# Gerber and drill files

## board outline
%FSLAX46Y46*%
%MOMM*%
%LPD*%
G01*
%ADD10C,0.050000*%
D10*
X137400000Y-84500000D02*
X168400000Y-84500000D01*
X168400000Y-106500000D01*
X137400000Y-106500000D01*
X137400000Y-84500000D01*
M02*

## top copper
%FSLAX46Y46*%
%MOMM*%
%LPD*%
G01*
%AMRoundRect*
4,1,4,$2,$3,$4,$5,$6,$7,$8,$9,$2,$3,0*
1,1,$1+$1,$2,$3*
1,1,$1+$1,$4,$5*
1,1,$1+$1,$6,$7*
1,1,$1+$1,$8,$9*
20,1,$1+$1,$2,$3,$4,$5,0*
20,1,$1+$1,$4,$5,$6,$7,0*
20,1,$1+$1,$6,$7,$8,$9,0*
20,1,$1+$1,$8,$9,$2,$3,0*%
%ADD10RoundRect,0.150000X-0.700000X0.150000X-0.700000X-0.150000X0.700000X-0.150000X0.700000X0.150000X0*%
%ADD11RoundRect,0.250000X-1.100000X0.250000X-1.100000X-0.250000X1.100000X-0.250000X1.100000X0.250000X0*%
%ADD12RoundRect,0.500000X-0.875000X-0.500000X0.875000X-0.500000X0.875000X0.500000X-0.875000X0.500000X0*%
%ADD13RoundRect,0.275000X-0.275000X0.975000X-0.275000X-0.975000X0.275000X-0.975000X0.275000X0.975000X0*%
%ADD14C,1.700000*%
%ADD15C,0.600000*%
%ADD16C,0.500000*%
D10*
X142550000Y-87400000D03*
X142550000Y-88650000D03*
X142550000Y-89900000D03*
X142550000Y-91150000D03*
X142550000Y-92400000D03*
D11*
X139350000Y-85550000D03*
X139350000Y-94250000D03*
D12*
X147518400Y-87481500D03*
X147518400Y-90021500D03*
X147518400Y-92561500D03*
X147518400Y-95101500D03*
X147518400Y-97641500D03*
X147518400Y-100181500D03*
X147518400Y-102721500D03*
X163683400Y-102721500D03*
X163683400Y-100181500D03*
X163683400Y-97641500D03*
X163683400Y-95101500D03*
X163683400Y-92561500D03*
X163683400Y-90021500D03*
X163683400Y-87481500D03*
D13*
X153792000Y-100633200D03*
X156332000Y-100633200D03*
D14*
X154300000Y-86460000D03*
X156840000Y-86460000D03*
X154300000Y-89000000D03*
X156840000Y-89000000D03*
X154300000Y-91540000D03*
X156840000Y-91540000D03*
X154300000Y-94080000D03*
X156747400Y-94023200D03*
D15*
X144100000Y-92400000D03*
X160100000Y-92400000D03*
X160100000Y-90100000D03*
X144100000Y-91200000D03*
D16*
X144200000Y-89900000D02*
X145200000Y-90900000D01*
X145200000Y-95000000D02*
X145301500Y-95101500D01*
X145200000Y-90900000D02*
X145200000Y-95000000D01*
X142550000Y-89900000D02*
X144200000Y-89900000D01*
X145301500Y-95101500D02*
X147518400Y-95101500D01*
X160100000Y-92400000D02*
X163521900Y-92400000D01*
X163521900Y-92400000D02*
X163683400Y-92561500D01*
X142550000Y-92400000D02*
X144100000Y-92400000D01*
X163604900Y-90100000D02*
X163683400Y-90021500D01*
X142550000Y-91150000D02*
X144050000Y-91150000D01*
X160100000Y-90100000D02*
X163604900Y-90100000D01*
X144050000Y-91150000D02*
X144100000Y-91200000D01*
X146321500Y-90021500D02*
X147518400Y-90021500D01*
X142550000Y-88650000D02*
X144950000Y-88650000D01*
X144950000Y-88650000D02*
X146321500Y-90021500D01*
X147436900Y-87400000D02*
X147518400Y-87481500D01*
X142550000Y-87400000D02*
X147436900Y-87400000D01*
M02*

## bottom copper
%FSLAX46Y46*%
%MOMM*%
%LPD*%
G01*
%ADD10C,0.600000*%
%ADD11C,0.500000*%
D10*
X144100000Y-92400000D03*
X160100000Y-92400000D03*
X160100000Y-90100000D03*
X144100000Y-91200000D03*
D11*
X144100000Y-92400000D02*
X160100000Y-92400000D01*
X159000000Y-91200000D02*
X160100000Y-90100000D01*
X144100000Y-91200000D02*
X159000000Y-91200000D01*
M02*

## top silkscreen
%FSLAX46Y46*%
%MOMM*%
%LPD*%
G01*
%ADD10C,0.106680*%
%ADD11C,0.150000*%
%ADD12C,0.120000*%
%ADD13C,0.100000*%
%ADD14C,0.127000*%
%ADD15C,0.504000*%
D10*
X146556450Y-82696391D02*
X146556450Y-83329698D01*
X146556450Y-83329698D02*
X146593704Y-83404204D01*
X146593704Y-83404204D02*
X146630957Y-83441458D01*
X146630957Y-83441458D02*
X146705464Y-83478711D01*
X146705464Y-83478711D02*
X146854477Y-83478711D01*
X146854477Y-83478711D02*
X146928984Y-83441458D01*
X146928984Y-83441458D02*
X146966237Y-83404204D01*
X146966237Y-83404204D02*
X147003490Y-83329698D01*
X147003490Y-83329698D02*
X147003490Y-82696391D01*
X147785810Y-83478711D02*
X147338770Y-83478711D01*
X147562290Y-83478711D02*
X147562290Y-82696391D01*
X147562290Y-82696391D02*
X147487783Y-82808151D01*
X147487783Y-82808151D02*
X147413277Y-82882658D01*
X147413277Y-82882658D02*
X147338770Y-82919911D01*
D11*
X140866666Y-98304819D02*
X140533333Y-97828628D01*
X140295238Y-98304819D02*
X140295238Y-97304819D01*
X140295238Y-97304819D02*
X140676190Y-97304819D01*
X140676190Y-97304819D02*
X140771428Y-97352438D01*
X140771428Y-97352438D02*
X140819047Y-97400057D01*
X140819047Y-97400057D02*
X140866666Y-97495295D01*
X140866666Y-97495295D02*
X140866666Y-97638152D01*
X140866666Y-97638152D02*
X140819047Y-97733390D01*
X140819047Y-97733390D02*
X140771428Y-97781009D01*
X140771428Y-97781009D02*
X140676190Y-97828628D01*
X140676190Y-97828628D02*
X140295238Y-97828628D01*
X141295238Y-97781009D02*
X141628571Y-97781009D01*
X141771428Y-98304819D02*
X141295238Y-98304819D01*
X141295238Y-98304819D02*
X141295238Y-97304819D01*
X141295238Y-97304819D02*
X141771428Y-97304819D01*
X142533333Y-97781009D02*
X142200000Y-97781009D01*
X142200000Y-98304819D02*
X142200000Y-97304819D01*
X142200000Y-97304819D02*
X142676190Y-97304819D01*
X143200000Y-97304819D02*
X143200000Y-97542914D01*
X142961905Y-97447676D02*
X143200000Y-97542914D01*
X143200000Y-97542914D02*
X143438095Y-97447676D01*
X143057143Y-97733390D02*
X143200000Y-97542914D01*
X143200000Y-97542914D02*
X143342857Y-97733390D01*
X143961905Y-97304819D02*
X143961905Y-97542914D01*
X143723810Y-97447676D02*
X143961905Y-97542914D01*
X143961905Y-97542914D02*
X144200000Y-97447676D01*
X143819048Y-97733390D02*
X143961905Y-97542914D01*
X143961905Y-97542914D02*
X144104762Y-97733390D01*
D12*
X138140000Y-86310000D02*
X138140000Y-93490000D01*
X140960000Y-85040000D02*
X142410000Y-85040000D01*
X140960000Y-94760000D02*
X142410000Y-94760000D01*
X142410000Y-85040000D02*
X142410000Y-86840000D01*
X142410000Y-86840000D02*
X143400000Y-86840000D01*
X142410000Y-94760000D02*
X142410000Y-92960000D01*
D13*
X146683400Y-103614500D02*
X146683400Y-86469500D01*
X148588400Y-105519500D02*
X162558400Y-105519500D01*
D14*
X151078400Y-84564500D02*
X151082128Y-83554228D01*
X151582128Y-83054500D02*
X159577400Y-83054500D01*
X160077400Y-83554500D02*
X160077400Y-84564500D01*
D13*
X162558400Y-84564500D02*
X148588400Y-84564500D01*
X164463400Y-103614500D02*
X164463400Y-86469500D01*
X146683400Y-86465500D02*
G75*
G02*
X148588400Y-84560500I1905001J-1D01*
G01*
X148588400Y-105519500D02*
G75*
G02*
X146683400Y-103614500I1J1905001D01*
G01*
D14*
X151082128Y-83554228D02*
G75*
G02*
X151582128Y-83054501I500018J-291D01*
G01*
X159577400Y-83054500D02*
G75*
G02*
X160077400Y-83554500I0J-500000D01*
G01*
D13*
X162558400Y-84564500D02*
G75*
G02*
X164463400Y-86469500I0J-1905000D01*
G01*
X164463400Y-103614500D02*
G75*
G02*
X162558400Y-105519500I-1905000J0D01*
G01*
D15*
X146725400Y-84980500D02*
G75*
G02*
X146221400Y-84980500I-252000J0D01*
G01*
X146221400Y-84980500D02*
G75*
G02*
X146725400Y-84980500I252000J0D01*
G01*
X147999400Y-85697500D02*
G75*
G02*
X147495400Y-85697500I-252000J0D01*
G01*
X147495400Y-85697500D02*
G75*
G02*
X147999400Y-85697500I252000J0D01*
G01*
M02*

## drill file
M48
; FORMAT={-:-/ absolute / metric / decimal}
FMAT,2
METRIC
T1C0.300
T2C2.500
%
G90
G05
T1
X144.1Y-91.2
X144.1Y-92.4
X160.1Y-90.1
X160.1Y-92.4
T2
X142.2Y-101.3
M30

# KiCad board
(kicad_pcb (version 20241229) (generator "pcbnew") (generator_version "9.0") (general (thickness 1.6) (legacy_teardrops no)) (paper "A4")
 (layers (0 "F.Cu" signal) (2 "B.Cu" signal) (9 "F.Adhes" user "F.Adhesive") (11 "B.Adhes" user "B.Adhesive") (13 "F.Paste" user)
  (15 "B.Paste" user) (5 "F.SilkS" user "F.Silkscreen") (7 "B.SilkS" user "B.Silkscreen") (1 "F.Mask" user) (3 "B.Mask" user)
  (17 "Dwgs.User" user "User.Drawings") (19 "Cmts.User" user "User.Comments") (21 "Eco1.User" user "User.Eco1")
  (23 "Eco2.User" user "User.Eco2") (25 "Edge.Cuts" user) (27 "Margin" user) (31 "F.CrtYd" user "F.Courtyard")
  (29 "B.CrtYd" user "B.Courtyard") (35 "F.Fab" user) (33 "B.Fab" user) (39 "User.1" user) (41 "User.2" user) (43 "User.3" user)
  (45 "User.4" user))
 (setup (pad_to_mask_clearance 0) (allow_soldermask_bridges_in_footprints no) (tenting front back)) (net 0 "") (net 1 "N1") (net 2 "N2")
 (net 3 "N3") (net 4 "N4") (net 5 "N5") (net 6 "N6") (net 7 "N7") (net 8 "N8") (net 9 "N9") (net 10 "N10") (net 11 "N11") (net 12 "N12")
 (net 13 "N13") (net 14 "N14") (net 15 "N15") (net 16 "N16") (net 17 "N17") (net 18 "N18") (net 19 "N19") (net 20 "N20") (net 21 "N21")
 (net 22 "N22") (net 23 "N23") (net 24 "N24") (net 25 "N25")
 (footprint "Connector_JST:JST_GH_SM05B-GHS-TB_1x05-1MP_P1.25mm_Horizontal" (layer "F.Cu") (at 140.7 89.9 -90)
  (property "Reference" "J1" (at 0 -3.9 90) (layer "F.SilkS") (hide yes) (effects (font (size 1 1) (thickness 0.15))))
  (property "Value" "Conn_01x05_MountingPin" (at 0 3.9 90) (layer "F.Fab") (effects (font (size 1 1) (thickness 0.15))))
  (fp_line (start -3.59 2.56) (end 3.59 2.56) (stroke (width 0.12) (type solid)) (layer "F.SilkS"))
  (fp_line (start -4.86 -0.26) (end -4.86 -1.71) (stroke (width 0.12) (type solid)) (layer "F.SilkS"))
  (fp_line (start 4.86 -0.26) (end 4.86 -1.71) (stroke (width 0.12) (type solid)) (layer "F.SilkS"))
  (fp_line (start -4.86 -1.71) (end -3.06 -1.71) (stroke (width 0.12) (type solid)) (layer "F.SilkS"))
  (fp_line (start -3.06 -1.71) (end -3.06 -2.7) (stroke (width 0.12) (type solid)) (layer "F.SilkS"))
  (fp_line (start 4.86 -1.71) (end 3.06 -1.71) (stroke (width 0.12) (type solid)) (layer "F.SilkS"))
  (pad "1" smd roundrect (at -2.5 -1.85 270) (size 0.6 1.7) (layers "F.Cu" "F.Mask" "F.Paste") (roundrect_rratio 0.25) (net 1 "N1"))
  (pad "2" smd roundrect (at -1.25 -1.85 270) (size 0.6 1.7) (layers "F.Cu" "F.Mask" "F.Paste") (roundrect_rratio 0.25) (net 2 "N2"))
  (pad "3" smd roundrect (at 0 -1.85 270) (size 0.6 1.7) (layers "F.Cu" "F.Mask" "F.Paste") (roundrect_rratio 0.25) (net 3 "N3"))
  (pad "4" smd roundrect (at 1.25 -1.85 270) (size 0.6 1.7) (layers "F.Cu" "F.Mask" "F.Paste") (roundrect_rratio 0.25) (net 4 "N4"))
  (pad "5" smd roundrect (at 2.5 -1.85 270) (size 0.6 1.7) (layers "F.Cu" "F.Mask" "F.Paste") (roundrect_rratio 0.25) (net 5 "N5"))
  (pad "MP" smd roundrect (at -4.35 1.35 270) (size 1 2.7) (layers "F.Cu" "F.Mask" "F.Paste") (roundrect_rratio 0.25) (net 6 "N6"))
  (pad "MP" smd roundrect (at 4.35 1.35 270) (size 1 2.7) (layers "F.Cu" "F.Mask" "F.Paste") (roundrect_rratio 0.25) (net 6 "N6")))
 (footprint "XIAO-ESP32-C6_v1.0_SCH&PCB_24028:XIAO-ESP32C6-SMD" (layer "F.Cu") (at 155.8 95.08)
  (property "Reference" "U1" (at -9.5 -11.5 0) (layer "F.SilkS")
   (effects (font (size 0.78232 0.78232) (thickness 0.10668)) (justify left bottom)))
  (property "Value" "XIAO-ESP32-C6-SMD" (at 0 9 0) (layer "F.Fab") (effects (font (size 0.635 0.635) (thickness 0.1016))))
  (fp_line (start -9.1166 8.5345) (end -9.1166 -8.6105) (stroke (width 0.1) (type solid)) (layer "F.SilkS"))
  (fp_line (start -7.2116 10.4395) (end 6.7584 10.4395) (stroke (width 0.1) (type solid)) (layer "F.SilkS"))
  (fp_line (start -4.7216 -10.5155) (end -4.717872 -11.525772) (stroke (width 0.127) (type solid)) (layer "F.SilkS"))
  (fp_line (start -4.217872 -12.0255) (end 3.7774 -12.0255) (stroke (width 0.127) (type solid)) (layer "F.SilkS"))
  (fp_line (start 4.2774 -11.5255) (end 4.2774 -10.5155) (stroke (width 0.127) (type solid)) (layer "F.SilkS"))
  (fp_line (start 6.7584 -10.5155) (end -7.2116 -10.5155) (stroke (width 0.1) (type solid)) (layer "F.SilkS"))
  (fp_line (start 8.6634 8.5345) (end 8.6634 -8.6105) (stroke (width 0.1) (type solid)) (layer "F.SilkS"))
  (fp_arc (start -9.1166 -8.6145) (mid -8.558638 -9.961538) (end -7.2116 -10.5195) (stroke (width 0.1) (type solid)) (layer "F.SilkS"))
  (fp_arc (start -7.2116 10.4395) (mid -8.558638 9.881538) (end -9.1166 8.5345) (stroke (width 0.1) (type solid)) (layer "F.SilkS"))
  (fp_arc (start -4.717872 -11.525772) (mid -4.571324 -11.879144) (end -4.217872 -12.0255) (stroke (width 0.127) (type default))
   (layer "F.SilkS"))
  (fp_arc (start 3.7774 -12.0255) (mid 4.130953 -11.879053) (end 4.2774 -11.5255) (stroke (width 0.127) (type default)) (layer "F.SilkS"))
  (fp_arc (start 6.7584 -10.5155) (mid 8.105438 -9.957538) (end 8.6634 -8.6105) (stroke (width 0.1) (type solid)) (layer "F.SilkS"))
  (fp_arc (start 8.6634 8.5345) (mid 8.105438 9.881538) (end 6.7584 10.4395) (stroke (width 0.1) (type solid)) (layer "F.SilkS"))
  (fp_circle (center -9.3266 -10.0995) (end -9.3266 -10.3535) (stroke (width 0.5) (type solid)) (fill yes) (layer "F.SilkS"))
  (fp_circle (center -8.0526 -9.3825) (end -8.0526 -9.6365) (stroke (width 0.5) (type solid)) (fill yes) (layer "F.SilkS"))
  (pad "1" smd roundrect (at -8.2816 -7.5985) (size 2.75 2) (layers "F.Cu" "F.Mask" "F.Paste") (roundrect_rratio 0.25) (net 1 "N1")
   (solder_mask_margin 0.0508) (thermal_bridge_angle 45))
  (pad "2" smd roundrect (at -8.2816 -5.0585) (size 2.75 2) (layers "F.Cu" "F.Mask" "F.Paste") (roundrect_rratio 0.25) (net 2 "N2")
   (solder_mask_margin 0.0508) (thermal_bridge_angle 45))
  (pad "3" smd roundrect (at -8.2816 -2.5185) (size 2.75 2) (layers "F.Cu" "F.Mask" "F.Paste") (roundrect_rratio 0.25) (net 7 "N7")
   (solder_mask_margin 0.0508) (thermal_bridge_angle 45))
  (pad "4" smd roundrect (at -8.2816 0.0215) (size 2.75 2) (layers "F.Cu" "F.Mask" "F.Paste") (roundrect_rratio 0.25) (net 3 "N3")
   (solder_mask_margin 0.0508) (thermal_bridge_angle 45))
  (pad "5" smd roundrect (at -8.2816 2.5615) (size 2.75 2) (layers "F.Cu" "F.Mask" "F.Paste") (roundrect_rratio 0.25) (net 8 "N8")
   (solder_mask_margin 0.0508) (thermal_bridge_angle 45))
  (pad "6" smd roundrect (at -8.2816 5.1015) (size 2.75 2) (layers "F.Cu" "F.Mask" "F.Paste") (roundrect_rratio 0.25) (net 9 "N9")
   (solder_mask_margin 0.0508) (thermal_bridge_angle 45))
  (pad "7" smd roundrect (at -8.2816 7.6415) (size 2.75 2) (layers "F.Cu" "F.Mask" "F.Paste") (roundrect_rratio 0.25) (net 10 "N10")
   (solder_mask_margin 0.0508) (thermal_bridge_angle 45))
  (pad "8" smd roundrect (at 7.8834 7.6415) (size 2.75 2) (layers "F.Cu" "F.Mask" "F.Paste") (roundrect_rratio 0.25) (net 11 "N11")
   (solder_mask_margin 0.0508) (thermal_bridge_angle 45))
  (pad "9" smd roundrect (at 7.8834 5.1015) (size 2.75 2) (layers "F.Cu" "F.Mask" "F.Paste") (roundrect_rratio 0.25) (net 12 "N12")
   (solder_mask_margin 0.0508) (thermal_bridge_angle 45))
  (pad "10" smd roundrect (at 7.8834 2.5615) (size 2.75 2) (layers "F.Cu" "F.Mask" "F.Paste") (roundrect_rratio 0.25) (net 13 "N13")
   (solder_mask_margin 0.0508) (thermal_bridge_angle 45))
  (pad "11" smd roundrect (at 7.8834 0.0215) (size 2.75 2) (layers "F.Cu" "F.Mask" "F.Paste") (roundrect_rratio 0.25) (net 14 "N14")
   (solder_mask_margin 0.0508) (thermal_bridge_angle 45))
  (pad "12" smd roundrect (at 7.8834 -2.5185) (size 2.75 2) (layers "F.Cu" "F.Mask" "F.Paste") (roundrect_rratio 0.25) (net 5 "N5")
   (solder_mask_margin 0.0508) (thermal_bridge_angle 45))
  (pad "13" smd roundrect (at 7.8834 -5.0585) (size 2.75 2) (layers "F.Cu" "F.Mask" "F.Paste") (roundrect_rratio 0.25) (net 4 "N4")
   (solder_mask_margin 0.0508) (thermal_bridge_angle 45))
  (pad "14" smd roundrect (at 7.8834 -7.5985) (size 2.75 2) (layers "F.Cu" "F.Mask" "F.Paste") (roundrect_rratio 0.25) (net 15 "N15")
   (solder_mask_margin 0.0508) (thermal_bridge_angle 45))
  (pad "15" smd roundrect (at -2.008 5.5532 270) (size 2.5 1.1) (layers "F.Cu" "F.Mask" "F.Paste") (roundrect_rratio 0.25) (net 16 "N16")
   (solder_mask_margin 0.0508) (thermal_bridge_angle 45))
  (pad "16" smd roundrect (at 0.532 5.5532 270) (size 2.5 1.1) (layers "F.Cu" "F.Mask" "F.Paste") (roundrect_rratio 0.25) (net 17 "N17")
   (solder_mask_margin 0.0508) (thermal_bridge_angle 45))
  (pad "17" smd circle (at -1.5 -8.62) (size 1.7 1.7) (layers "F.Cu" "F.Mask" "F.Paste") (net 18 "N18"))
  (pad "18" smd circle (at 1.04 -8.62) (size 1.7 1.7) (layers "F.Cu" "F.Mask" "F.Paste") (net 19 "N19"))
  (pad "19" smd circle (at -1.5 -6.08) (size 1.7 1.7) (layers "F.Cu" "F.Mask" "F.Paste") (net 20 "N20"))
  (pad "20" smd circle (at 1.04 -6.08) (size 1.7 1.7) (layers "F.Cu" "F.Mask" "F.Paste") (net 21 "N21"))
  (pad "21" smd circle (at -1.5 -3.54) (size 1.7 1.7) (layers "F.Cu" "F.Mask" "F.Paste") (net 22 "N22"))
  (pad "22" smd circle (at 1.04 -3.54) (size 1.7 1.7) (layers "F.Cu" "F.Mask" "F.Paste") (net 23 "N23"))
  (pad "23" smd circle (at -1.5 -1) (size 1.7 1.7) (layers "F.Cu" "F.Mask" "F.Paste") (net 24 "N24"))
  (pad "24" smd circle (at 0.9474 -1.0568) (size 1.7 1.7) (layers "F.Cu" "F.Mask" "F.Paste") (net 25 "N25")))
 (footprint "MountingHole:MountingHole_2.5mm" (layer "F.Cu") (at 142.2 101.3)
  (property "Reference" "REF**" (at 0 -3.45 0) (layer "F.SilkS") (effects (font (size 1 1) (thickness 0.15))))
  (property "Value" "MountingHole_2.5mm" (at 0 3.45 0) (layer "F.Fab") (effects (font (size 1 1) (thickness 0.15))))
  (pad "" np_thru_hole circle (at 0 0) (size 2.5 2.5) (drill 2.5) (layers "*.Cu" "*.Mask")))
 (gr_rect (start 137.4 84.5) (end 168.4 106.5) (stroke (width 0.05) (type solid)) (fill no) (layer "Edge.Cuts"))
 (segment (start 144.2 89.9) (end 145.2 90.9) (width 0.5) (layer "F.Cu") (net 3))
 (segment (start 145.2 95) (end 145.3015 95.1015) (width 0.5) (layer "F.Cu") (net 3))
 (segment (start 145.2 90.9) (end 145.2 95) (width 0.5) (layer "F.Cu") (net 3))
 (segment (start 142.55 89.9) (end 144.2 89.9) (width 0.5) (layer "F.Cu") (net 3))
 (segment (start 145.3015 95.1015) (end 147.5184 95.1015) (width 0.5) (layer "F.Cu") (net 3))
 (segment (start 160.1 92.4) (end 163.5219 92.4) (width 0.5) (layer "F.Cu") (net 5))
 (segment (start 163.5219 92.4) (end 163.6834 92.5615) (width 0.5) (layer "F.Cu") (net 5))
 (segment (start 142.55 92.4) (end 144.1 92.4) (width 0.5) (layer "F.Cu") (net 5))
 (via (at 144.1 92.4) (size 0.6) (drill 0.3) (layers "F.Cu" "B.Cu") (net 5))
 (via (at 160.1 92.4) (size 0.6) (drill 0.3) (layers "F.Cu" "B.Cu") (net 5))
 (segment (start 144.1 92.4) (end 160.1 92.4) (width 0.5) (layer "B.Cu") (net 5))
 (segment (start 163.6049 90.1) (end 163.6834 90.0215) (width 0.5) (layer "F.Cu") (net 4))
 (segment (start 142.55 91.15) (end 144.05 91.15) (width 0.5) (layer "F.Cu") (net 4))
 (segment (start 160.1 90.1) (end 163.6049 90.1) (width 0.5) (layer "F.Cu") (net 4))
 (segment (start 144.05 91.15) (end 144.1 91.2) (width 0.5) (layer "F.Cu") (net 4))
 (via (at 160.1 90.1) (size 0.6) (drill 0.3) (layers "F.Cu" "B.Cu") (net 4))
 (via (at 144.1 91.2) (size 0.6) (drill 0.3) (layers "F.Cu" "B.Cu") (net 4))
 (segment (start 159 91.2) (end 160.1 90.1) (width 0.5) (layer "B.Cu") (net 4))
 (segment (start 144.1 91.2) (end 159 91.2) (width 0.5) (layer "B.Cu") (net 4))
 (segment (start 146.3215 90.0215) (end 147.5184 90.0215) (width 0.5) (layer "F.Cu") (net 2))
 (segment (start 142.55 88.65) (end 144.95 88.65) (width 0.5) (layer "F.Cu") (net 2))
 (segment (start 144.95 88.65) (end 146.3215 90.0215) (width 0.5) (layer "F.Cu") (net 2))
 (segment (start 147.4369 87.4) (end 147.5184 87.4815) (width 0.5) (layer "F.Cu") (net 1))
 (segment (start 142.55 87.4) (end 147.4369 87.4) (width 0.5) (layer "F.Cu") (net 1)))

